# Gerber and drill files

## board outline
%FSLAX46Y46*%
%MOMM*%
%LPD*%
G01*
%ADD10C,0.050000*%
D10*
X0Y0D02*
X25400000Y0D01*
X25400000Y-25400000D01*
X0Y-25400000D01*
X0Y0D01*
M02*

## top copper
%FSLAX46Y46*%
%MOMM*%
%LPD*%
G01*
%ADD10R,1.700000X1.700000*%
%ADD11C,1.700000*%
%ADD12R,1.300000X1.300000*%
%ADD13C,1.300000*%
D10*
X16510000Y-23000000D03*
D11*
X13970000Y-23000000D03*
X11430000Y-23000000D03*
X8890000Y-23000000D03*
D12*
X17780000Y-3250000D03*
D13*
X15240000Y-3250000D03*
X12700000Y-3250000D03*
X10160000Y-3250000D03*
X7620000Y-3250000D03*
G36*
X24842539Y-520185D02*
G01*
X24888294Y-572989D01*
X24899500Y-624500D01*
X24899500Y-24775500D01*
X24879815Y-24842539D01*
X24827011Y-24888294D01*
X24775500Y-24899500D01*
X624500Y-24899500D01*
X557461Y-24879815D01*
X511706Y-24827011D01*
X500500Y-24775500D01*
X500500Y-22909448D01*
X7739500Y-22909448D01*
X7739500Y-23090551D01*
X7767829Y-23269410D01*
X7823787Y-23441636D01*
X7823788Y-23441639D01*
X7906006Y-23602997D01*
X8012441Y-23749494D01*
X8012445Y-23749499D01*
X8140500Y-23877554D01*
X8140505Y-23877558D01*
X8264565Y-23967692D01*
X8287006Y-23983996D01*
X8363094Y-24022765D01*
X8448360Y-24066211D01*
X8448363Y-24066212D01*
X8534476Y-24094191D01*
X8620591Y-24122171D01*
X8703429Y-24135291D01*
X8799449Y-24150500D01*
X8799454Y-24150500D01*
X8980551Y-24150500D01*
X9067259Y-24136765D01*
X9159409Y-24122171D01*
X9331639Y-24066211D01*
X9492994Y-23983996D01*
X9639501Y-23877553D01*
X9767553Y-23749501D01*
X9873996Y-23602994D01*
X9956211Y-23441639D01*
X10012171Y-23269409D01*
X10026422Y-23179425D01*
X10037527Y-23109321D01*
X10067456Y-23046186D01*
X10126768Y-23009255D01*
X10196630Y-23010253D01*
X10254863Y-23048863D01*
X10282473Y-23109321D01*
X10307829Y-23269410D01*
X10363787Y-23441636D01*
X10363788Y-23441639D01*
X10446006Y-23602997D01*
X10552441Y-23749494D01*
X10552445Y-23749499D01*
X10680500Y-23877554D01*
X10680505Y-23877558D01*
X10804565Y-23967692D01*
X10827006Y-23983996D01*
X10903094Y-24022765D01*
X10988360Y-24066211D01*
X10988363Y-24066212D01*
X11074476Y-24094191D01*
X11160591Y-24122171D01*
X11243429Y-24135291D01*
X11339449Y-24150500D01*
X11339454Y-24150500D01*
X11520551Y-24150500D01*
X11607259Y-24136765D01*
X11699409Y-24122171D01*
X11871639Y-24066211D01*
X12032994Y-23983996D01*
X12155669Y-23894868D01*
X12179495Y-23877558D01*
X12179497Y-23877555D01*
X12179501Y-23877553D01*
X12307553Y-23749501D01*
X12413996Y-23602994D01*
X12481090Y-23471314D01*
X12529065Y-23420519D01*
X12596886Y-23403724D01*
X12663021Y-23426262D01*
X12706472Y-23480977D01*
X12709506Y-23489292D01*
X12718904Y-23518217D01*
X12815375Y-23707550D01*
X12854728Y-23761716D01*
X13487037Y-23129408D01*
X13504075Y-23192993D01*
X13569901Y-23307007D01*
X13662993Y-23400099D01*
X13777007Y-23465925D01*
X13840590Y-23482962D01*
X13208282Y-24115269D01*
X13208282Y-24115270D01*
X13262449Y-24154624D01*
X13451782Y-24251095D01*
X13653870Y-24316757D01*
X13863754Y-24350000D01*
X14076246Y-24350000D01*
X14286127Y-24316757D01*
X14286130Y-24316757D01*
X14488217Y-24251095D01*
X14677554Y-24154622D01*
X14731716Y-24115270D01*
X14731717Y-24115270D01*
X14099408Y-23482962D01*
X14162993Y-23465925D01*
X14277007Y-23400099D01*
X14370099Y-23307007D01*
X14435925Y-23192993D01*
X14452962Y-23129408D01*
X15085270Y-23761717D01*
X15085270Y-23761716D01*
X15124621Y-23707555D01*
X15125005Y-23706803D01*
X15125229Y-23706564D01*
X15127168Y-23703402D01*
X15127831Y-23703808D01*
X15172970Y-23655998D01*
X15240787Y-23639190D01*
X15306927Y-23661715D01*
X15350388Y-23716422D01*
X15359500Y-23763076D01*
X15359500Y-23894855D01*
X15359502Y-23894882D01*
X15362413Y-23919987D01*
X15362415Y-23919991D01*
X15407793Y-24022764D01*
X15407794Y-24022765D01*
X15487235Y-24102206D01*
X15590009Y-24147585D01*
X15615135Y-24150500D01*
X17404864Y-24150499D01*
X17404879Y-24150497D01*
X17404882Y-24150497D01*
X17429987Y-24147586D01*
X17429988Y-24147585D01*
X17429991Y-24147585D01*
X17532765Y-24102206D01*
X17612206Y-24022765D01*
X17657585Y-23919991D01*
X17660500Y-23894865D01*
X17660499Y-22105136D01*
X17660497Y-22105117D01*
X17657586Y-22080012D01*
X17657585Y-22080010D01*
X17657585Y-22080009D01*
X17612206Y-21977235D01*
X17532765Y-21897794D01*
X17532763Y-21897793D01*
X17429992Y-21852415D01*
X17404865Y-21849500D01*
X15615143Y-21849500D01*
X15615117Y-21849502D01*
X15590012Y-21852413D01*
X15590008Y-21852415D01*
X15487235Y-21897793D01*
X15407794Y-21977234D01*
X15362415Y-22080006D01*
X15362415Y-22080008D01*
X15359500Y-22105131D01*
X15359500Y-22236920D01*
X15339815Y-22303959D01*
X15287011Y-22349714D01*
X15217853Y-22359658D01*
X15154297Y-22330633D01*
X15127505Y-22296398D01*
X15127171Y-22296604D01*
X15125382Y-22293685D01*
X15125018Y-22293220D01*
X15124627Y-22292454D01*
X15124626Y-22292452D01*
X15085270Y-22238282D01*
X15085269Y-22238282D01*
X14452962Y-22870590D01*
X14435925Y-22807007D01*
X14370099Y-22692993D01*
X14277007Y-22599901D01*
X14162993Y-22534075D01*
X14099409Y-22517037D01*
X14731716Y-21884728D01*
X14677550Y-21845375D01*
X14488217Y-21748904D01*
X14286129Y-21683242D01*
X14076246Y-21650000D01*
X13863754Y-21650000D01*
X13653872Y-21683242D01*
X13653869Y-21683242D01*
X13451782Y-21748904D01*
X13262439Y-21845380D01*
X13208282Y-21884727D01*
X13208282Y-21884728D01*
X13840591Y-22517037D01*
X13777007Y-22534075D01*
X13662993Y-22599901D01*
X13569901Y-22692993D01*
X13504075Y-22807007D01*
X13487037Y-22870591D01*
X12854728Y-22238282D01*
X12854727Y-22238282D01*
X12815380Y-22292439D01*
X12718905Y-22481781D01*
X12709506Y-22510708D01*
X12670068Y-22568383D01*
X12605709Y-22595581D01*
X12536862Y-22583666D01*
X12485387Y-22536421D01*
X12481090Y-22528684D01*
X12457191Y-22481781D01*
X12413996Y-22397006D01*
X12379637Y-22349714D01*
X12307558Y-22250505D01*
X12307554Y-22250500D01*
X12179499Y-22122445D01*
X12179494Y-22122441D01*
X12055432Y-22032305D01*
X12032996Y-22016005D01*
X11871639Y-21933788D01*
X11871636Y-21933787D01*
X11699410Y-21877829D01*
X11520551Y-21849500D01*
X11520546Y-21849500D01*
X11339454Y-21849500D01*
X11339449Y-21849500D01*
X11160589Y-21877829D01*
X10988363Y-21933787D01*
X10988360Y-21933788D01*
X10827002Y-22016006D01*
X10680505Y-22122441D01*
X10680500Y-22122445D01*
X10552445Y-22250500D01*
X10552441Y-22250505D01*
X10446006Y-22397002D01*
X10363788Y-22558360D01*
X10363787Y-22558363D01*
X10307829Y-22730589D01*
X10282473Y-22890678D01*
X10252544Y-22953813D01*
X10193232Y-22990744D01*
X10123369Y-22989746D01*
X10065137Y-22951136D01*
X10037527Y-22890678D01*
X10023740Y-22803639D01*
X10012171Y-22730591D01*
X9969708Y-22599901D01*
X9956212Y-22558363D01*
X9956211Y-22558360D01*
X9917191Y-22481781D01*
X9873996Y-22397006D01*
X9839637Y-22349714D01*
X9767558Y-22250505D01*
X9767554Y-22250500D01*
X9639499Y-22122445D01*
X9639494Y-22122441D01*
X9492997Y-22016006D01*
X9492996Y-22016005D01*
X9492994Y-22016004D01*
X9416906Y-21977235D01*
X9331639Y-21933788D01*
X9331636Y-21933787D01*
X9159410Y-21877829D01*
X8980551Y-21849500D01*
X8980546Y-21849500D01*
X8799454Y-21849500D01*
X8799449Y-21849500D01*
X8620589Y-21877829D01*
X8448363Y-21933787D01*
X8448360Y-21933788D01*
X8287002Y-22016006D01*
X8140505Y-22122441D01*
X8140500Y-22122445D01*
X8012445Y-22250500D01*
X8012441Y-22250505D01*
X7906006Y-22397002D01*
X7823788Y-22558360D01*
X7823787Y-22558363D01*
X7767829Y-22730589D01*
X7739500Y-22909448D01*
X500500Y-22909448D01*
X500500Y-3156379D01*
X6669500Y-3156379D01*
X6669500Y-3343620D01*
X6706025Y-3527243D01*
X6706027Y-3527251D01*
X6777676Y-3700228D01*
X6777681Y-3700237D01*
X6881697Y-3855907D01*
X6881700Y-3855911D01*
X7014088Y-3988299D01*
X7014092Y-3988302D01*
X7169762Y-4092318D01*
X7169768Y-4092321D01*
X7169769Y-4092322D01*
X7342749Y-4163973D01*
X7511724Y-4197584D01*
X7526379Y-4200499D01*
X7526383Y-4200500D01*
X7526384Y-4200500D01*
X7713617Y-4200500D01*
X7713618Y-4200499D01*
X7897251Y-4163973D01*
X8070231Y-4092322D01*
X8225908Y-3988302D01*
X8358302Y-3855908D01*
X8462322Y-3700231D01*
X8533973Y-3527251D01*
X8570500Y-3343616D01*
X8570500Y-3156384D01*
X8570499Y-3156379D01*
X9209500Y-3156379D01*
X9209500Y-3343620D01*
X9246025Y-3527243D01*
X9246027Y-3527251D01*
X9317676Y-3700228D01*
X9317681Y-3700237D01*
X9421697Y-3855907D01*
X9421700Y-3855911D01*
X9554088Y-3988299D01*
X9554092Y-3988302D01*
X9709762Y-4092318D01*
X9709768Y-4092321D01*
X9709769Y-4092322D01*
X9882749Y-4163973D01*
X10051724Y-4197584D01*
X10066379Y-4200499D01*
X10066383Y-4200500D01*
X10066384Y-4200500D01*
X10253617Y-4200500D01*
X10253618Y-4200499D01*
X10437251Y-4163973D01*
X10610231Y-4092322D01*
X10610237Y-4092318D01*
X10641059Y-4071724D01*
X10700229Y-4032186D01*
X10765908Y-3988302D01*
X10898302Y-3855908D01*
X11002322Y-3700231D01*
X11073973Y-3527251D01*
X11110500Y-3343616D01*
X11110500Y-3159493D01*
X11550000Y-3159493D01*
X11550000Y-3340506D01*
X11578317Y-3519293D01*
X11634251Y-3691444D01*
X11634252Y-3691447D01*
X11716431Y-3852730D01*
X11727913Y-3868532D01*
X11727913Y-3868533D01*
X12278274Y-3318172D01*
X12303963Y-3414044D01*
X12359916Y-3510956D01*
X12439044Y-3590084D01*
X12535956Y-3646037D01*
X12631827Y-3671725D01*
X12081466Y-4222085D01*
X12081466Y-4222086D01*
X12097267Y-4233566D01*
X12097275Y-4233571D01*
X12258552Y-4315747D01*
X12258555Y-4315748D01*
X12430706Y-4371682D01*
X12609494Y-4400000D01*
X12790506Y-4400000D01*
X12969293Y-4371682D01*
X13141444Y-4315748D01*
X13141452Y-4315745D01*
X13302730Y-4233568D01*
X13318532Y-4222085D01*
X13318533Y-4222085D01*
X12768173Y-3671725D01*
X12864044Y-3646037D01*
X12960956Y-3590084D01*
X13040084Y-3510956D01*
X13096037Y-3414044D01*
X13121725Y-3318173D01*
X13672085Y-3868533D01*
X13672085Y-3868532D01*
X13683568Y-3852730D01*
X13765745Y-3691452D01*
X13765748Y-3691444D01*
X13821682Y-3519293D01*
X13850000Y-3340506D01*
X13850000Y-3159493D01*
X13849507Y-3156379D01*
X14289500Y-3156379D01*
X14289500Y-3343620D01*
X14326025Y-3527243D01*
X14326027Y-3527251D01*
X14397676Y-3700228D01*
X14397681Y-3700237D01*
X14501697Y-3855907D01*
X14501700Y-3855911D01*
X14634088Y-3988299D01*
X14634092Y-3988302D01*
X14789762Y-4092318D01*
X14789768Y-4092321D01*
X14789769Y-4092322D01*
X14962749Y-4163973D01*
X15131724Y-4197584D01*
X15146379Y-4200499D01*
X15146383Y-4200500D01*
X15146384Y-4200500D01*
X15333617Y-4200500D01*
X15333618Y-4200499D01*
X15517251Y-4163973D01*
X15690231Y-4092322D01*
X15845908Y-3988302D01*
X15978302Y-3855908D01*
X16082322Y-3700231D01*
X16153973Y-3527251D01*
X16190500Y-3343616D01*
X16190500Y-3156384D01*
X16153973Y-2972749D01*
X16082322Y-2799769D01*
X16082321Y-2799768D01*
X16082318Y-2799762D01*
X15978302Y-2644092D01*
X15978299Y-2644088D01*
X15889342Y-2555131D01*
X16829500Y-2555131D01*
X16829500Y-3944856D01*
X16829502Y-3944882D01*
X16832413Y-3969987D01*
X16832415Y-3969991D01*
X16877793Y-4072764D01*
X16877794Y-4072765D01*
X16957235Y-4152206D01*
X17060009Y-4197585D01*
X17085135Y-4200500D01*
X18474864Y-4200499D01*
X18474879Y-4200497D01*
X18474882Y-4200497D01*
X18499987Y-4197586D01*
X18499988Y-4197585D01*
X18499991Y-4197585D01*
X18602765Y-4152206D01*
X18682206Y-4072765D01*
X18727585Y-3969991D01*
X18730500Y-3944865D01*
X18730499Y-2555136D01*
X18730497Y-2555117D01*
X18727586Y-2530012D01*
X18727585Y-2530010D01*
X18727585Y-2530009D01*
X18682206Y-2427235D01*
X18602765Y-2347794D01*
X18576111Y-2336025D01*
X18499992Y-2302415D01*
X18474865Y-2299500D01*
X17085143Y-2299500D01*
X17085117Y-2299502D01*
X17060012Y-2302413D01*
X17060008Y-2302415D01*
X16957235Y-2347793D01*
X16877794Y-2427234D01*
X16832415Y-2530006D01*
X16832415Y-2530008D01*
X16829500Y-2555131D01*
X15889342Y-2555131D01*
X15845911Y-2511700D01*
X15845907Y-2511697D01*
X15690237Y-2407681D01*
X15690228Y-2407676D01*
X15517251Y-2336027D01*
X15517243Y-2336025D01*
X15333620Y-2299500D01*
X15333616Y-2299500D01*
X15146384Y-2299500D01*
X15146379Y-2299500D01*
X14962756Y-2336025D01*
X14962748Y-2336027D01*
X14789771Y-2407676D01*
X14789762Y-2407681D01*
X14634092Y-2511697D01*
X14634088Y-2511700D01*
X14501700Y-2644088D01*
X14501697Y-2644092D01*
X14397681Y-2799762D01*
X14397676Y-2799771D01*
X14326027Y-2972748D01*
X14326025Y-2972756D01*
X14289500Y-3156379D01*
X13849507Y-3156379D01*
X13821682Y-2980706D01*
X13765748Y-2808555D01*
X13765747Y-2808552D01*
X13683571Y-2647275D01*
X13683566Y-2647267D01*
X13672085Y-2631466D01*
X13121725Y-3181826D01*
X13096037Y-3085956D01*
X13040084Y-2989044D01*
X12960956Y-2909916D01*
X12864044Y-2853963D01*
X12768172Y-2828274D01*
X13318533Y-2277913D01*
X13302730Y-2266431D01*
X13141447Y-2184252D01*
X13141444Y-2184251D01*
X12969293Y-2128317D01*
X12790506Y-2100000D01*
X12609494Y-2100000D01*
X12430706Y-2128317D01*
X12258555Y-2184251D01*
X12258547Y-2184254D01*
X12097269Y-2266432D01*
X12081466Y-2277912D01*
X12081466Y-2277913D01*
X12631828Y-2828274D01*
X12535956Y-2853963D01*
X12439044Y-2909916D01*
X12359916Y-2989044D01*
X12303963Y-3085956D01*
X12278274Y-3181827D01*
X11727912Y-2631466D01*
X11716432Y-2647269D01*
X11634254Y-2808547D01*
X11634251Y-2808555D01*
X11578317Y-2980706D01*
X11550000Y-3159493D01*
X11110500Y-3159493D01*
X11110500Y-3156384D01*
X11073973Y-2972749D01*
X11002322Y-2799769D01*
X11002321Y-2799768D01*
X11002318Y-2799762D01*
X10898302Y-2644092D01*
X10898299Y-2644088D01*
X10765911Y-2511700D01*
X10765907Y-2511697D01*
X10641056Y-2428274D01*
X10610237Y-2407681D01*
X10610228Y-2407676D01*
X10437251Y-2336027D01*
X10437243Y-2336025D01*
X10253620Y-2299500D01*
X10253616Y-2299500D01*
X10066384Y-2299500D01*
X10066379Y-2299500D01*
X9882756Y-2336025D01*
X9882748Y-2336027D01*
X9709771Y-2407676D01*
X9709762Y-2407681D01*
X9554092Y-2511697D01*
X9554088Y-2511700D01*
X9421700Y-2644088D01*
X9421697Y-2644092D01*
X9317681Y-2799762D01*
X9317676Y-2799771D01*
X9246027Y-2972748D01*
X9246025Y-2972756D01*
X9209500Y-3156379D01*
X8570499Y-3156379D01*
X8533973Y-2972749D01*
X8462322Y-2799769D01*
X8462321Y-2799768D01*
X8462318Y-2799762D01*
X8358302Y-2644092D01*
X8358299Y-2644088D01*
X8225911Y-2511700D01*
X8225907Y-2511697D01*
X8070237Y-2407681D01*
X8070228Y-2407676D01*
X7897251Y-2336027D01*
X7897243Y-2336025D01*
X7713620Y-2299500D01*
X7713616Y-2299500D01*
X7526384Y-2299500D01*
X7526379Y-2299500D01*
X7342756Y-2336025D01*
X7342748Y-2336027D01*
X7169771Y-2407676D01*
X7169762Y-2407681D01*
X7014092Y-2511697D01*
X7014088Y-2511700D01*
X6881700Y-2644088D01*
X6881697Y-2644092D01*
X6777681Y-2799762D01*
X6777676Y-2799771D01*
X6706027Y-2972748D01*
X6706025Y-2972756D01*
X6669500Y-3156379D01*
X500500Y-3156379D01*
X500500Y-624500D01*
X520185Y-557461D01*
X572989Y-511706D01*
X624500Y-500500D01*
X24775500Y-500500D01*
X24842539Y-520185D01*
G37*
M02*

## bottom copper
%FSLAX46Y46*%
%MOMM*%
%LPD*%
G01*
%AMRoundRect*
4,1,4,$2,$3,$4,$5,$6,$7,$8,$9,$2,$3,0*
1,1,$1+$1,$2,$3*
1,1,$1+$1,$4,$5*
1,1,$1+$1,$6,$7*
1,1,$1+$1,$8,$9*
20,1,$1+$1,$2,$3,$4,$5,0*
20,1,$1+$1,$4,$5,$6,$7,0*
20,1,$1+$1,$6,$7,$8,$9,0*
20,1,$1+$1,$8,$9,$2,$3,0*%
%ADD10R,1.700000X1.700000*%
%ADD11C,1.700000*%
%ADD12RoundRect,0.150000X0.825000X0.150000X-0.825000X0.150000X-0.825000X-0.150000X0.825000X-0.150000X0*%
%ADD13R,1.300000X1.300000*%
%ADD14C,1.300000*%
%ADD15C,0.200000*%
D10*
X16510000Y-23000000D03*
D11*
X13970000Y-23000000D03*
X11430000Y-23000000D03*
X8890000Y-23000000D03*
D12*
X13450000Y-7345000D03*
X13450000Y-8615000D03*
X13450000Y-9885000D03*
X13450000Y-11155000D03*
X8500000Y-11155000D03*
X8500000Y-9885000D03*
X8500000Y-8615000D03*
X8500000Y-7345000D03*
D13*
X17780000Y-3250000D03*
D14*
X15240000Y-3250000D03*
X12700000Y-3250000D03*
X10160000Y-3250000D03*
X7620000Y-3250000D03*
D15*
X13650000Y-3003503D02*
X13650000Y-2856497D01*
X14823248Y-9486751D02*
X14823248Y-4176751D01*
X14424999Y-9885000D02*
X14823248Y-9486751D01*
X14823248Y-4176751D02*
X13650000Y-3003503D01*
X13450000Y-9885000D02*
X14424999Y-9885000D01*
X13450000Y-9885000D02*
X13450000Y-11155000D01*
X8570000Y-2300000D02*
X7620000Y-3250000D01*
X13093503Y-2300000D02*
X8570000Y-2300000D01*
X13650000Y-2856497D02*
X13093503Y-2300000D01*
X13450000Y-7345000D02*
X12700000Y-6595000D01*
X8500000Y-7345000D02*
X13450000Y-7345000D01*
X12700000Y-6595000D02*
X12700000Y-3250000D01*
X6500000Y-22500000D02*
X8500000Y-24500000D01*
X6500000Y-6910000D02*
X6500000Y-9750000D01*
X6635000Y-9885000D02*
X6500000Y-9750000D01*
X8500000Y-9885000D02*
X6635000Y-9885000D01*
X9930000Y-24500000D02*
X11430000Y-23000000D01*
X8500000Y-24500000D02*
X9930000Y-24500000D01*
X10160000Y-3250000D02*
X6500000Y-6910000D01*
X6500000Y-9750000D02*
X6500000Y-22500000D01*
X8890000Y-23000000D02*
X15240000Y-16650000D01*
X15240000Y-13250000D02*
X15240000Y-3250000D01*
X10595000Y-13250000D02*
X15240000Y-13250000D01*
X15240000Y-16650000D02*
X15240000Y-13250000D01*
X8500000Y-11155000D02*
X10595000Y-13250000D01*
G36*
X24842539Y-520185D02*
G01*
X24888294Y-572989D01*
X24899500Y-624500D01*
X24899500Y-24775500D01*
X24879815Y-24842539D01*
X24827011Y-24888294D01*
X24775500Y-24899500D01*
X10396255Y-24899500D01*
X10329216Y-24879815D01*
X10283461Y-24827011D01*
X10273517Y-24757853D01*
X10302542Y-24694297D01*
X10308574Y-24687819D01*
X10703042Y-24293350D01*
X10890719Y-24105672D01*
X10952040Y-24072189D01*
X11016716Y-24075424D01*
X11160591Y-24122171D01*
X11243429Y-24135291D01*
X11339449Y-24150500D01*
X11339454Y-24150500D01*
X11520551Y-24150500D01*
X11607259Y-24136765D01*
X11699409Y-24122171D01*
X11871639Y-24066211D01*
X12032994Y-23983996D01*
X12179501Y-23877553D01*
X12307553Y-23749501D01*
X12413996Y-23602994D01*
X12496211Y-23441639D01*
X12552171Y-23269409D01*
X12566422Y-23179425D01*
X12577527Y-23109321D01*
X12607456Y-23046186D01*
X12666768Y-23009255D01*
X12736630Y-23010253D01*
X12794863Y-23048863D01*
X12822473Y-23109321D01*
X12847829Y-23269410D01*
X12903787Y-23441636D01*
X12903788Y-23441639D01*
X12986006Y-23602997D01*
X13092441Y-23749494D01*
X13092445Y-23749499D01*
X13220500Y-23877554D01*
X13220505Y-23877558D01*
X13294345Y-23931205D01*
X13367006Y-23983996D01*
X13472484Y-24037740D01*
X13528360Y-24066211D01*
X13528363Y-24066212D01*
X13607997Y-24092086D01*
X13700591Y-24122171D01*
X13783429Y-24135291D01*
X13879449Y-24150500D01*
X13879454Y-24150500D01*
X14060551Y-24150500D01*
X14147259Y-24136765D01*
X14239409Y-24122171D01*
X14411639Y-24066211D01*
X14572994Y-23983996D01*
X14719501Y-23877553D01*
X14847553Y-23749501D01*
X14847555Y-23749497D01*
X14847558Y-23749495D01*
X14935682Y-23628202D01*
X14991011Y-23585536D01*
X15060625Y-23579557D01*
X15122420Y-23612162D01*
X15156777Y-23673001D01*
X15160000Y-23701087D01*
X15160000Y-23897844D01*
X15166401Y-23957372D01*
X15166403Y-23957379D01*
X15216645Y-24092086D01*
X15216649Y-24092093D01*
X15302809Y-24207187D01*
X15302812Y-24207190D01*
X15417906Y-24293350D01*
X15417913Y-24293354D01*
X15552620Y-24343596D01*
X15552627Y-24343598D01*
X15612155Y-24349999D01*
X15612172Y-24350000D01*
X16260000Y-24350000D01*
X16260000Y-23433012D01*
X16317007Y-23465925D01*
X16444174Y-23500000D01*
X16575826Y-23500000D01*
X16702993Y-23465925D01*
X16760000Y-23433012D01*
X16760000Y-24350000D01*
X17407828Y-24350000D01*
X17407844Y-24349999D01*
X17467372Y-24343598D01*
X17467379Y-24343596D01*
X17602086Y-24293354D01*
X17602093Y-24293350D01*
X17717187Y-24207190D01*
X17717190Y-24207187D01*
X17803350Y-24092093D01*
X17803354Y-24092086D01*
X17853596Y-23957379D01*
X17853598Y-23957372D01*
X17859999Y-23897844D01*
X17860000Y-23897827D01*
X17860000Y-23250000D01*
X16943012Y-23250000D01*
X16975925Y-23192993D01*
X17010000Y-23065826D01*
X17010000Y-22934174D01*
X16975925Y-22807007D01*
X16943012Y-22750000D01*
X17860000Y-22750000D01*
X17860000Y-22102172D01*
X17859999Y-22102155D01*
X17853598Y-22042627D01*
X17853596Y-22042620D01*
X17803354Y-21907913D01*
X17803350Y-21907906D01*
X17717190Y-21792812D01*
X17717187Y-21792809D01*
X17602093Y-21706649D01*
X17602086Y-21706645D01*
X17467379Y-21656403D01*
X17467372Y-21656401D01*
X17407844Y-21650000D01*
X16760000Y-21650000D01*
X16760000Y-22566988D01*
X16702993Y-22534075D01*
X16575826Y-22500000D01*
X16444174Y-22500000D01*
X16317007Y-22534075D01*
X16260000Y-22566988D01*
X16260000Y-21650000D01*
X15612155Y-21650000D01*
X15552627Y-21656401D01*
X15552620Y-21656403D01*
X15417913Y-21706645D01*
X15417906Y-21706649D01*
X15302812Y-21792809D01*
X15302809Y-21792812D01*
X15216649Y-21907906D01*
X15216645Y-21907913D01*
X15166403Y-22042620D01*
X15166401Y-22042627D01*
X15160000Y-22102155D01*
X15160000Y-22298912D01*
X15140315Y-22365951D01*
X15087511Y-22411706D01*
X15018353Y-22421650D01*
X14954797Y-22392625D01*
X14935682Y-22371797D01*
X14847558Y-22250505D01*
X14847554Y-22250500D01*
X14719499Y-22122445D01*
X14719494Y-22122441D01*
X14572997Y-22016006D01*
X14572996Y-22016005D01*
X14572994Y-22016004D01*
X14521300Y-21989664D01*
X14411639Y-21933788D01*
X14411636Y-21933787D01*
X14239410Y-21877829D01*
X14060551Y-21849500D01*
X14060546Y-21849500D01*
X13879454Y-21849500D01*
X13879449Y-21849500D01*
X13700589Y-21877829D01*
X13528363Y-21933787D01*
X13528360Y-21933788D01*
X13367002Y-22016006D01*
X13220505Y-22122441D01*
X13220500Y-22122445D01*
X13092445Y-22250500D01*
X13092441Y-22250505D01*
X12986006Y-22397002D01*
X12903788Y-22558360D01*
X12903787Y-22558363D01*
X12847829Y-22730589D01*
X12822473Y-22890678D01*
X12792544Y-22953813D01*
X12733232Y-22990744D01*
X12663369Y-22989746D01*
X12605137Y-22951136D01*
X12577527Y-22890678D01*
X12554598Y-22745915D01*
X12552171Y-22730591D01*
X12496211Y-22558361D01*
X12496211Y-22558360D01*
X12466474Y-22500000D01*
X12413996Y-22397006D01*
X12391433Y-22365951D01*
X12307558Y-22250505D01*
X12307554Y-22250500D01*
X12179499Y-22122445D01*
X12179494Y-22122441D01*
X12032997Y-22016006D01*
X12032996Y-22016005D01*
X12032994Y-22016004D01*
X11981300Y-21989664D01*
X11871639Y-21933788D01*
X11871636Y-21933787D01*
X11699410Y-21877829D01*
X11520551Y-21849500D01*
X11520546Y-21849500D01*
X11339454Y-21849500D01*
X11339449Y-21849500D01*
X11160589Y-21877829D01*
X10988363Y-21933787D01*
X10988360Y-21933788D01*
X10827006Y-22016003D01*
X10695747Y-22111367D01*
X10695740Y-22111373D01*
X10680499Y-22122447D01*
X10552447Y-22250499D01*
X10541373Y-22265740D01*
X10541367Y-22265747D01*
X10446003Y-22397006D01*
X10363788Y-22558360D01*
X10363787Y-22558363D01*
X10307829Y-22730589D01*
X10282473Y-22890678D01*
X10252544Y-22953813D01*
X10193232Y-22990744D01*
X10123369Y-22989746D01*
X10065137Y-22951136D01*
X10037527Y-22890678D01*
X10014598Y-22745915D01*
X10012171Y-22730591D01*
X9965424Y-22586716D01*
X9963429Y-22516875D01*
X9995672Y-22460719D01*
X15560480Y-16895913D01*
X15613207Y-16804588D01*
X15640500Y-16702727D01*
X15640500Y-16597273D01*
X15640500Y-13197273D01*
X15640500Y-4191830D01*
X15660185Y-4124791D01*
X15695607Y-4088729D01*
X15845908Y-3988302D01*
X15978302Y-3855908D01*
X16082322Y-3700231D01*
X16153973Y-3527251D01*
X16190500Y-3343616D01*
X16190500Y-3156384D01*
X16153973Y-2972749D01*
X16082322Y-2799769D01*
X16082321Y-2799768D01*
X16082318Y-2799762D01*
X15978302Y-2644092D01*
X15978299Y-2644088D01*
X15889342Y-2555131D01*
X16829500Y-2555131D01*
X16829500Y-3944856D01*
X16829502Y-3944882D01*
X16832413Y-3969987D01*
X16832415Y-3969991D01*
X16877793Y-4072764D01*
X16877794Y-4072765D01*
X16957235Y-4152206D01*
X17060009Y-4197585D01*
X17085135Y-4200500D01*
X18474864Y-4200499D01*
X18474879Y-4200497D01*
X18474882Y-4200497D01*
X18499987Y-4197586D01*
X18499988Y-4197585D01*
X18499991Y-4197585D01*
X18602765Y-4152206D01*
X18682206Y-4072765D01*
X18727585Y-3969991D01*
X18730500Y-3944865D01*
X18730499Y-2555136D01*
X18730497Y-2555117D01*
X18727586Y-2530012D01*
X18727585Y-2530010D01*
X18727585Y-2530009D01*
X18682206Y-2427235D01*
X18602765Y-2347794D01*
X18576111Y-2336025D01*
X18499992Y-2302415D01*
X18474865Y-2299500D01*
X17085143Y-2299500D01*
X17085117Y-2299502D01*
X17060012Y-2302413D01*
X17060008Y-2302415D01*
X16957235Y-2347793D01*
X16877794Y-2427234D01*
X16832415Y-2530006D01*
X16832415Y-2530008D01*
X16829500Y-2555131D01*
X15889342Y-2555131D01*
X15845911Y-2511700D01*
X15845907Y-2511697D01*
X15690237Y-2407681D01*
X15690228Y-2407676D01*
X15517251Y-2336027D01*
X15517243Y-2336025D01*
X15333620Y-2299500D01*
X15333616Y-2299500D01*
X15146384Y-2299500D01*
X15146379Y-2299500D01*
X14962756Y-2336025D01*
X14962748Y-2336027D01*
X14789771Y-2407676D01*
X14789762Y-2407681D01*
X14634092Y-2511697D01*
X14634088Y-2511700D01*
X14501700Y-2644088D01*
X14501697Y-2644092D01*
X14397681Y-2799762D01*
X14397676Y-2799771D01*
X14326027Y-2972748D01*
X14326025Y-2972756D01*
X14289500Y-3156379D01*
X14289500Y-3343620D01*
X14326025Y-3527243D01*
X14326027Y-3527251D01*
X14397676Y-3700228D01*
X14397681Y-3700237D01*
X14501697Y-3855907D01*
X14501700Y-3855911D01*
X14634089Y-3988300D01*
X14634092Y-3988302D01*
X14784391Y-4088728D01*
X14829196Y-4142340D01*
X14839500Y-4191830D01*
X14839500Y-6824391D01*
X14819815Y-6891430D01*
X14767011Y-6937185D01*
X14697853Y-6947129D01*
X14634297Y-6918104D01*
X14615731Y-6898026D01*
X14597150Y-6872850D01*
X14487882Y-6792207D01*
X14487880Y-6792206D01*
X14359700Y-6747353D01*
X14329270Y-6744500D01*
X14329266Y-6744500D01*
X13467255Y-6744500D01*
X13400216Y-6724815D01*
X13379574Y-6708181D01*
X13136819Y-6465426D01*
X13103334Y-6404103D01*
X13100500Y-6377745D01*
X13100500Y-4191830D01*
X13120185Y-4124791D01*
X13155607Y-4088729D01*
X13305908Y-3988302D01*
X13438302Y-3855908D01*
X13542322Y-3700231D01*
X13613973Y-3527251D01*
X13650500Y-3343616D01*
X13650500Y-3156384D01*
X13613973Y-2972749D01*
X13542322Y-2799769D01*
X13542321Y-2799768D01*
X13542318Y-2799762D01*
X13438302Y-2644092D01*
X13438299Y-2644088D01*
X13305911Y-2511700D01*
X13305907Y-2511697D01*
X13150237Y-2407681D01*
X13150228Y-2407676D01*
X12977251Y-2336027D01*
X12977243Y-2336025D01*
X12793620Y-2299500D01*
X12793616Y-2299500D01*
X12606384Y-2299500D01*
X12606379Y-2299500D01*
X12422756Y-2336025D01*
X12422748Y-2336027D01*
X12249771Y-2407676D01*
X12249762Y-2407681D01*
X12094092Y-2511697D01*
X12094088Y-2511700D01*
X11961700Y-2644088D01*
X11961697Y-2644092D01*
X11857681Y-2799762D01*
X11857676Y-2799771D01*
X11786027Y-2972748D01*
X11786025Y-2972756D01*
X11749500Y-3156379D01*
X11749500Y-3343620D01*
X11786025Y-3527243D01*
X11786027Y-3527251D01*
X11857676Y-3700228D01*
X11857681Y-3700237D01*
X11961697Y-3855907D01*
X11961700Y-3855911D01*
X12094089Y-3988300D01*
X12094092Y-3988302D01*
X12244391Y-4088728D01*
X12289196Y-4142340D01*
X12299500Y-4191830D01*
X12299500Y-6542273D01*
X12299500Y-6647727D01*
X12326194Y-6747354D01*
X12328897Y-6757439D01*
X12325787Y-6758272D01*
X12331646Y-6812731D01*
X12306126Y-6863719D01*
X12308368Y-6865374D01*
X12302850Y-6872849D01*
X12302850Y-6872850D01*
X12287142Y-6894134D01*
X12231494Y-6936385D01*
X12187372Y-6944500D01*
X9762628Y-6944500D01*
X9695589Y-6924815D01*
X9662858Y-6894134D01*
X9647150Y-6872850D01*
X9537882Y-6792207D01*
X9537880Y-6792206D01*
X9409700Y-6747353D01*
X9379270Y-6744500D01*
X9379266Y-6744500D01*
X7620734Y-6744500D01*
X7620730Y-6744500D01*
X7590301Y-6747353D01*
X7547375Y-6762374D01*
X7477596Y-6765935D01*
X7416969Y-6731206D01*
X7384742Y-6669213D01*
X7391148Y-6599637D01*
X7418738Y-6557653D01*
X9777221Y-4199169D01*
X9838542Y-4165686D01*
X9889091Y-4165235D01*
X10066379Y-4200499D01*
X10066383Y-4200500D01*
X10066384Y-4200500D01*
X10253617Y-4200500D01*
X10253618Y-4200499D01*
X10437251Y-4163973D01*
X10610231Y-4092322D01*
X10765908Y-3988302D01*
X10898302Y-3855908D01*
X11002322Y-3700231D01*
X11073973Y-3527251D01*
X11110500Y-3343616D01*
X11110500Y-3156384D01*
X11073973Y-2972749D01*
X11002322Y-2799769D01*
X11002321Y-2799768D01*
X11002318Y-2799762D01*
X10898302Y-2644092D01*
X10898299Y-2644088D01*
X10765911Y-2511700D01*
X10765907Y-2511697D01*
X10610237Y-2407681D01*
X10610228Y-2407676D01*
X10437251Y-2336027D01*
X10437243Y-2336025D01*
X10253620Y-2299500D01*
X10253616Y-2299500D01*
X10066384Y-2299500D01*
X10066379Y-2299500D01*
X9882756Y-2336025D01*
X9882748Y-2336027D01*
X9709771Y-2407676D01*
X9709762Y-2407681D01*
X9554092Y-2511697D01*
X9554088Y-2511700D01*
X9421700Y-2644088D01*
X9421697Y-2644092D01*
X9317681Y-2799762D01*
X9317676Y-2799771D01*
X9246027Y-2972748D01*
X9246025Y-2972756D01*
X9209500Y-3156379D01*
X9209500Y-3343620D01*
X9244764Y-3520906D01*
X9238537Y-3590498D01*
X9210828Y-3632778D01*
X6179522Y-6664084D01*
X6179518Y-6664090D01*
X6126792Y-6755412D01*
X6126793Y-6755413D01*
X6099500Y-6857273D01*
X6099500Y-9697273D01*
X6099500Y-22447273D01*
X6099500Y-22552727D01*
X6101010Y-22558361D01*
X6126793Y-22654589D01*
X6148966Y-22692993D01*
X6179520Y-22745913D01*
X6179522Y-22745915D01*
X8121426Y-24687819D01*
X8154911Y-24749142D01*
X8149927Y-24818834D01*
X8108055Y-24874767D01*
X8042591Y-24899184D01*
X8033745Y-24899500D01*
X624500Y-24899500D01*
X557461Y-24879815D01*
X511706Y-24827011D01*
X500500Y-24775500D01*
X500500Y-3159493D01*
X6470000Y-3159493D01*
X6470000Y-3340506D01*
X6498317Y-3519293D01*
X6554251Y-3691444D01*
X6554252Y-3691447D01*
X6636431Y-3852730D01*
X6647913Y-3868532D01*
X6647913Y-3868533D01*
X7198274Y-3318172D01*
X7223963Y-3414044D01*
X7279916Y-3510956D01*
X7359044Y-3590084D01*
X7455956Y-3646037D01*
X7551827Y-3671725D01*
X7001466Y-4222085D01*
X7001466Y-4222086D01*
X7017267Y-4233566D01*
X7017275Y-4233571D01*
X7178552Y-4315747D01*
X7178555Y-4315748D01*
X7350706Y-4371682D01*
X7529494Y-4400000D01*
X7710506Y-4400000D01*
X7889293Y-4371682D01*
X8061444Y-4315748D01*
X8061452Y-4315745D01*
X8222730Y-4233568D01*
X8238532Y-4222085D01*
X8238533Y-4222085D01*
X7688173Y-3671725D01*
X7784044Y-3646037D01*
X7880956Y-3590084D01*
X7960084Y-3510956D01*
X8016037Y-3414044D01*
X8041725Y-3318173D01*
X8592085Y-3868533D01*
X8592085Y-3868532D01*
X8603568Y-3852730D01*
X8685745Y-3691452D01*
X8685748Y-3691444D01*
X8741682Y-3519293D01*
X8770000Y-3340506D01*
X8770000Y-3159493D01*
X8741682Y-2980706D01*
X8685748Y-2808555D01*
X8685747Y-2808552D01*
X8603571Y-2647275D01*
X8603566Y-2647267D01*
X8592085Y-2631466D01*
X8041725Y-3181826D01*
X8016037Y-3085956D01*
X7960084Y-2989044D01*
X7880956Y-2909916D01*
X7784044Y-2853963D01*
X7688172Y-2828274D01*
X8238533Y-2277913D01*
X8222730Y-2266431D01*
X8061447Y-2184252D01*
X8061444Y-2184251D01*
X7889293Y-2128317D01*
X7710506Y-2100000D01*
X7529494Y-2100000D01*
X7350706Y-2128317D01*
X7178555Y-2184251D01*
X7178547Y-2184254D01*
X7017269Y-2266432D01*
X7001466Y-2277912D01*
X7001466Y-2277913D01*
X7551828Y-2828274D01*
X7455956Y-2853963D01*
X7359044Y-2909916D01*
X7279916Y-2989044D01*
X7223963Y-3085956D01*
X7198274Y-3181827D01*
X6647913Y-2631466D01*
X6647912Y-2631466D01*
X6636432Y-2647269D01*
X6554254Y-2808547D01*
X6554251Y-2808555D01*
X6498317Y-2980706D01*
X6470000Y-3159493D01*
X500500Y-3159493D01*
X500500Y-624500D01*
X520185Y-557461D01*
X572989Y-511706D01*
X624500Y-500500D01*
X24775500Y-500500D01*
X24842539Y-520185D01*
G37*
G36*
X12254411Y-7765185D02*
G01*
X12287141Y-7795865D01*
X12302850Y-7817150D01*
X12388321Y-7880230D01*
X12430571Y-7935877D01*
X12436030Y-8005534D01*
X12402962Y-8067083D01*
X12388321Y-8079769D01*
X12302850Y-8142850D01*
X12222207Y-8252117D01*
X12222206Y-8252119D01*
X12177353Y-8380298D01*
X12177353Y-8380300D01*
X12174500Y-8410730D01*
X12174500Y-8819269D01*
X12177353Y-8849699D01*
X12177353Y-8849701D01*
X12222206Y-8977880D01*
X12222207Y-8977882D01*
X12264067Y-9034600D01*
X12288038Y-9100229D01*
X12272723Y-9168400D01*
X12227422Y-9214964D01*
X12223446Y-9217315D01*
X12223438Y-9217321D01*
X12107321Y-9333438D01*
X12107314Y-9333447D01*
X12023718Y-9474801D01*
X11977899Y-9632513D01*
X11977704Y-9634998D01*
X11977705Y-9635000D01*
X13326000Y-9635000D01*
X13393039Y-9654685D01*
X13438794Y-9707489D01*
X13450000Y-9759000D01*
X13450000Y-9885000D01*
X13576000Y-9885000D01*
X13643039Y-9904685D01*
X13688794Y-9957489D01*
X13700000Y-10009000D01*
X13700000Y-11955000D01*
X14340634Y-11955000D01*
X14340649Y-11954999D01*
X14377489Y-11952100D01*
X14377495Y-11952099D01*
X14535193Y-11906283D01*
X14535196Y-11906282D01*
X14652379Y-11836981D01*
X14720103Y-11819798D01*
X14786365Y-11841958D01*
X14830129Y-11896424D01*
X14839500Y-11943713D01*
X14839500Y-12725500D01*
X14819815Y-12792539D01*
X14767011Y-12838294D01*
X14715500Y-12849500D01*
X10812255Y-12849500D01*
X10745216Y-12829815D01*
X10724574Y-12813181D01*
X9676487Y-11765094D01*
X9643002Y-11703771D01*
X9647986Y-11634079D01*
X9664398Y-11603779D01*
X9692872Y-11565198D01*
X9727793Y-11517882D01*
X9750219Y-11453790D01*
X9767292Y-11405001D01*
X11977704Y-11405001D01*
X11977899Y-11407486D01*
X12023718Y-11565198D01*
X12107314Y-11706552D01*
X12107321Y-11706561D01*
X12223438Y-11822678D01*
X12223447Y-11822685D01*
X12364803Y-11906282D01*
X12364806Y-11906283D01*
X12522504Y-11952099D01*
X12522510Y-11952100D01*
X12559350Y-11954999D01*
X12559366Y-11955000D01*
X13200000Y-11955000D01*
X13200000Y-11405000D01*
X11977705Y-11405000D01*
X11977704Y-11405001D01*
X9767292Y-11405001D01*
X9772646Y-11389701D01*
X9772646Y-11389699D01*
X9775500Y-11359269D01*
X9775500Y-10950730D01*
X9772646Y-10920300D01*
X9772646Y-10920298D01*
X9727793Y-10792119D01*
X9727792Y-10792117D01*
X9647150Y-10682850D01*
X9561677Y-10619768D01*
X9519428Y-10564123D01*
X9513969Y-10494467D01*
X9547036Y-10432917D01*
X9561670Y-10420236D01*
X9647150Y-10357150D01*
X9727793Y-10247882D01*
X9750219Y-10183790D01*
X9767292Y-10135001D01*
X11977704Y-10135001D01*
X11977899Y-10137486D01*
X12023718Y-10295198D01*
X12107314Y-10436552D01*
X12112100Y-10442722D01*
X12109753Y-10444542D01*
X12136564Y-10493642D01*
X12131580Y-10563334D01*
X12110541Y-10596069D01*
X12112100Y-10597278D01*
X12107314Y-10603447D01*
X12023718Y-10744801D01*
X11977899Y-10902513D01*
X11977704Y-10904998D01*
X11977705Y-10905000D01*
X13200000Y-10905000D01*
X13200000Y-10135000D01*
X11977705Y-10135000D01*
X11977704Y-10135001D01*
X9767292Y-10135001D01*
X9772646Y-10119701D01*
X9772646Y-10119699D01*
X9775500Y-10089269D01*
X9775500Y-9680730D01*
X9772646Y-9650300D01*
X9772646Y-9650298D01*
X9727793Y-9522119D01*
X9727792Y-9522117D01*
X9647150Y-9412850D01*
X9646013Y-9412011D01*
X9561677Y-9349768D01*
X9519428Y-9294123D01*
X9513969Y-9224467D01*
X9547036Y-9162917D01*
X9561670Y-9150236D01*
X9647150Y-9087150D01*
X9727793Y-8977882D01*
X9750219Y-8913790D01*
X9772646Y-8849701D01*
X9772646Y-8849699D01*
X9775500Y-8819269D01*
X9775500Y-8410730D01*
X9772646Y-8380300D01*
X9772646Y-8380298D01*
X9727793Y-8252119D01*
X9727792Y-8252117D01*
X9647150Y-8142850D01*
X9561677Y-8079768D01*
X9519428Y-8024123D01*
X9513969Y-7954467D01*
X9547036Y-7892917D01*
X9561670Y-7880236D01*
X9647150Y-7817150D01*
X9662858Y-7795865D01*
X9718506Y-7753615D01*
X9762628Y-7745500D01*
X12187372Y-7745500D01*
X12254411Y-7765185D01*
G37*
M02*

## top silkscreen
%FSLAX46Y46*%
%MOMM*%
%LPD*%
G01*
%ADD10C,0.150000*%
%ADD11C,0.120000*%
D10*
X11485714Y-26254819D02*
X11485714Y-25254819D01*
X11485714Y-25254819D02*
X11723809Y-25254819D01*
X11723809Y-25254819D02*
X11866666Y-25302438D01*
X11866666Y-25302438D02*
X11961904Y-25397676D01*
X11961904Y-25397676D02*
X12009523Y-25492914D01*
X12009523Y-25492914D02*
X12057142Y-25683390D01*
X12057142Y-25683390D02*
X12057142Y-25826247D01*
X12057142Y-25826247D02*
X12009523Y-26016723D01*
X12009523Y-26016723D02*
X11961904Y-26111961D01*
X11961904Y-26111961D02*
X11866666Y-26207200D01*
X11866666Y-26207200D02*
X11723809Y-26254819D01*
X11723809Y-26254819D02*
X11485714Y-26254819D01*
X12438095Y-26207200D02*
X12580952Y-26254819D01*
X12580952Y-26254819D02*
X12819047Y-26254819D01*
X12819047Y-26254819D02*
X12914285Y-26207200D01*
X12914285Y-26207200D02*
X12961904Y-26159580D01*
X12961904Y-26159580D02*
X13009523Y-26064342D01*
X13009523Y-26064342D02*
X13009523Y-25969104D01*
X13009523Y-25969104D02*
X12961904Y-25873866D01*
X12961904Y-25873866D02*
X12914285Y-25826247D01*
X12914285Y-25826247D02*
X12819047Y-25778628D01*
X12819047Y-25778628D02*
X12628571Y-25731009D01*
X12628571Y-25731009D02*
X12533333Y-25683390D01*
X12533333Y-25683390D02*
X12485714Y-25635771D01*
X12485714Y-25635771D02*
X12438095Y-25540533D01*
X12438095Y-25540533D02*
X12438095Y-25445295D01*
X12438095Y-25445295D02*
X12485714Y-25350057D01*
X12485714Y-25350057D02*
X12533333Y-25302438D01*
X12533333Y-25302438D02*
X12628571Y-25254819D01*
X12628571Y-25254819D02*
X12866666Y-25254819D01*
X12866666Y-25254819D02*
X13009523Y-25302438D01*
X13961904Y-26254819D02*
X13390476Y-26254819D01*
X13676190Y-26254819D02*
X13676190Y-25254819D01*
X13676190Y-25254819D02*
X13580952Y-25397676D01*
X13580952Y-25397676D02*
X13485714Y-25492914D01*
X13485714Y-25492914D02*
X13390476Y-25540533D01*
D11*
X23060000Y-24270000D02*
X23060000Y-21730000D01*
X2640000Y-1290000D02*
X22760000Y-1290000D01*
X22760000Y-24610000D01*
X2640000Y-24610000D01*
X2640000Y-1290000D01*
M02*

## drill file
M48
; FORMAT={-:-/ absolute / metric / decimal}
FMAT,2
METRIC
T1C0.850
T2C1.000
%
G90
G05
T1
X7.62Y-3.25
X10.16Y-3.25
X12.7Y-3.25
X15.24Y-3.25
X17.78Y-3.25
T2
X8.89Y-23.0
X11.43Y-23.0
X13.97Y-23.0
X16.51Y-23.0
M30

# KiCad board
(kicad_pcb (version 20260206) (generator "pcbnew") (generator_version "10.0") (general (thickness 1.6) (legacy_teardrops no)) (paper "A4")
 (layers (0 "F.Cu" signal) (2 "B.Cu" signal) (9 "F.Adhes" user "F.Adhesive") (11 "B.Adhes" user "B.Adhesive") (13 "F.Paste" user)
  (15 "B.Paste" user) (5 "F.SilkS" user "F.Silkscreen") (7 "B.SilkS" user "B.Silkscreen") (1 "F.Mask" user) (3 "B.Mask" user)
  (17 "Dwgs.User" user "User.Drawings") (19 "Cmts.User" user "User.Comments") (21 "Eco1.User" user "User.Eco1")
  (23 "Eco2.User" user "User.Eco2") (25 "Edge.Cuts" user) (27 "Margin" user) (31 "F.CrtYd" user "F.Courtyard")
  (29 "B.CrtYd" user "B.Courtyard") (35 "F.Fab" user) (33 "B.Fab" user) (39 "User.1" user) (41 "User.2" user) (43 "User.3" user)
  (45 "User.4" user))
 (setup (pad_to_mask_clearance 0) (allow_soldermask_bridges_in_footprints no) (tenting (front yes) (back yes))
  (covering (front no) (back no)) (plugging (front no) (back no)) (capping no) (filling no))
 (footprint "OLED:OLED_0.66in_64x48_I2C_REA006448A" (layer "F.Cu") (at 16.51 23 180)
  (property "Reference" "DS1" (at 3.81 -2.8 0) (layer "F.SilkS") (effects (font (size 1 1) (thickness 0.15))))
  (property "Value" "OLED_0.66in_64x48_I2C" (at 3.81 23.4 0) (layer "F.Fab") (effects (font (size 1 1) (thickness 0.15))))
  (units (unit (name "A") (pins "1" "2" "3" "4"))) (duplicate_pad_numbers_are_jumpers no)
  (fp_line (start -6.55 -1.27) (end -6.55 1.27) (stroke (width 0.12) (type solid)) (layer "F.SilkS"))
  (fp_rect (start -6.25 -1.61) (end 13.87 21.71) (stroke (width 0.12) (type solid)) (fill no) (layer "F.SilkS"))
  (pad "1" thru_hole rect (at 0 0 180) (size 1.7 1.7) (drill 1) (layers "*.Cu" "*.Mask") (remove_unused_layers no) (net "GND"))
  (pad "2" thru_hole circle (at 2.54 0 180) (size 1.7 1.7) (drill 1) (layers "*.Cu" "*.Mask") (remove_unused_layers no) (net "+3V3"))
  (pad "3" thru_hole circle (at 5.08 0 180) (size 1.7 1.7) (drill 1) (layers "*.Cu" "*.Mask") (remove_unused_layers no) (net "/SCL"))
  (pad "4" thru_hole circle (at 7.62 0 180) (size 1.7 1.7) (drill 1) (layers "*.Cu" "*.Mask") (remove_unused_layers no) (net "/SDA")))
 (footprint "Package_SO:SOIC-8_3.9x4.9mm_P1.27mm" (layer "B.Cu") (at 10.975 9.25 180)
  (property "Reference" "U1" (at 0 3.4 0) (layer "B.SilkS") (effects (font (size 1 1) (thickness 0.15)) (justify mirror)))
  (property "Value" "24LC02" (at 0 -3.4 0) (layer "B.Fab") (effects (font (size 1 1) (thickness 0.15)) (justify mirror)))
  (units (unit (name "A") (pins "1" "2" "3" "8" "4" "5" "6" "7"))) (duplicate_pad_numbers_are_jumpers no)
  (pad "1" smd roundrect (at -2.475 1.905 180) (size 1.95 0.6) (layers "B.Cu" "B.Mask" "B.Paste") (roundrect_rratio 0.25) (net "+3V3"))
  (pad "2" smd roundrect (at -2.475 0.635 180) (size 1.95 0.6) (layers "B.Cu" "B.Mask" "B.Paste") (roundrect_rratio 0.25)
   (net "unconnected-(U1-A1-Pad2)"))
  (pad "3" smd roundrect (at -2.475 -0.635 180) (size 1.95 0.6) (layers "B.Cu" "B.Mask" "B.Paste") (roundrect_rratio 0.25) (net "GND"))
  (pad "4" smd roundrect (at -2.475 -1.905 180) (size 1.95 0.6) (layers "B.Cu" "B.Mask" "B.Paste") (roundrect_rratio 0.25) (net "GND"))
  (pad "5" smd roundrect (at 2.475 -1.905 180) (size 1.95 0.6) (layers "B.Cu" "B.Mask" "B.Paste") (roundrect_rratio 0.25) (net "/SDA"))
  (pad "6" smd roundrect (at 2.475 -0.635 180) (size 1.95 0.6) (layers "B.Cu" "B.Mask" "B.Paste") (roundrect_rratio 0.25) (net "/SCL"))
  (pad "7" smd roundrect (at 2.475 0.635 180) (size 1.95 0.6) (layers "B.Cu" "B.Mask" "B.Paste") (roundrect_rratio 0.25)
   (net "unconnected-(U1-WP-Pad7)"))
  (pad "8" smd roundrect (at 2.475 1.905 180) (size 1.95 0.6) (layers "B.Cu" "B.Mask" "B.Paste") (roundrect_rratio 0.25) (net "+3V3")))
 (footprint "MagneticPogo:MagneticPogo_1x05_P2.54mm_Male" (layer "B.Cu") (at 12.7 3.25 180)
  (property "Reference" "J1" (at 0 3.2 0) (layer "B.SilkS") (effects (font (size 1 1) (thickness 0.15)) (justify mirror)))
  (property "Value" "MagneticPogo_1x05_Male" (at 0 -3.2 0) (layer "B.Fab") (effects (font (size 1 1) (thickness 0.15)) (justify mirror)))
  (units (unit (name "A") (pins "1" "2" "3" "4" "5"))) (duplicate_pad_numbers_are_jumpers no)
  (pad "1" thru_hole rect (at -5.08 0 180) (size 1.3 1.3) (drill 0.85) (layers "*.Cu" "*.Mask") (remove_unused_layers no) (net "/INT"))
  (pad "2" thru_hole circle (at -2.54 0 180) (size 1.3 1.3) (drill 0.85) (layers "*.Cu" "*.Mask") (remove_unused_layers no) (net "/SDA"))
  (pad "3" thru_hole circle (at 0 0 180) (size 1.3 1.3) (drill 0.85) (layers "*.Cu" "*.Mask") (remove_unused_layers no) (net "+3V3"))
  (pad "4" thru_hole circle (at 2.54 0 180) (size 1.3 1.3) (drill 0.85) (layers "*.Cu" "*.Mask") (remove_unused_layers no) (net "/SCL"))
  (pad "5" thru_hole circle (at 5.08 0 180) (size 1.3 1.3) (drill 0.85) (layers "*.Cu" "*.Mask") (remove_unused_layers no) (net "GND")))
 (gr_rect (start 0 0) (end 25.4 25.4) (stroke (width 0.05) (type default)) (fill no) (layer "Edge.Cuts"))
 (segment (start 13.65 3.003503) (end 13.65 2.856497) (width 0.2) (layer "B.Cu") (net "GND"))
 (segment (start 14.823248 9.486751) (end 14.823248 4.176751) (width 0.2) (layer "B.Cu") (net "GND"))
 (segment (start 14.424999 9.885) (end 14.823248 9.486751) (width 0.2) (layer "B.Cu") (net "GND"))
 (segment (start 14.823248 4.176751) (end 13.65 3.003503) (width 0.2) (layer "B.Cu") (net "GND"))
 (segment (start 13.45 9.885) (end 14.424999 9.885) (width 0.2) (layer "B.Cu") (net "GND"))
 (segment (start 13.45 9.885) (end 13.45 11.155) (width 0.2) (layer "B.Cu") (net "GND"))
 (segment (start 8.57 2.3) (end 7.62 3.25) (width 0.2) (layer "B.Cu") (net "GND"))
 (segment (start 13.093503 2.3) (end 8.57 2.3) (width 0.2) (layer "B.Cu") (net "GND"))
 (segment (start 13.65 2.856497) (end 13.093503 2.3) (width 0.2) (layer "B.Cu") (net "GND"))
 (segment (start 13.45 7.345) (end 12.7 6.595) (width 0.2) (layer "B.Cu") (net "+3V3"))
 (segment (start 8.5 7.345) (end 13.45 7.345) (width 0.2) (layer "B.Cu") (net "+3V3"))
 (segment (start 12.7 6.595) (end 12.7 3.25) (width 0.2) (layer "B.Cu") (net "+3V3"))
 (segment (start 6.5 22.5) (end 8.5 24.5) (width 0.2) (layer "B.Cu") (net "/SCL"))
 (segment (start 6.5 6.91) (end 6.5 9.75) (width 0.2) (layer "B.Cu") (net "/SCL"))
 (segment (start 6.635 9.885) (end 6.5 9.75) (width 0.2) (layer "B.Cu") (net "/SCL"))
 (segment (start 8.5 9.885) (end 6.635 9.885) (width 0.2) (layer "B.Cu") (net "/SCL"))
 (segment (start 9.93 24.5) (end 11.43 23) (width 0.2) (layer "B.Cu") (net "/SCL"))
 (segment (start 8.5 24.5) (end 9.93 24.5) (width 0.2) (layer "B.Cu") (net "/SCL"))
 (segment (start 10.16 3.25) (end 6.5 6.91) (width 0.2) (layer "B.Cu") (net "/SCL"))
 (segment (start 6.5 9.75) (end 6.5 22.5) (width 0.2) (layer "B.Cu") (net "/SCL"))
 (segment (start 8.89 23) (end 15.24 16.65) (width 0.2) (layer "B.Cu") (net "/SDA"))
 (segment (start 15.24 13.25) (end 15.24 3.25) (width 0.2) (layer "B.Cu") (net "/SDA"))
 (segment (start 10.595 13.25) (end 15.24 13.25) (width 0.2) (layer "B.Cu") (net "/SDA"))
 (segment (start 15.24 16.65) (end 15.24 13.25) (width 0.2) (layer "B.Cu") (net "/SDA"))
 (segment (start 8.5 11.155) (end 10.595 13.25) (width 0.2) (layer "B.Cu") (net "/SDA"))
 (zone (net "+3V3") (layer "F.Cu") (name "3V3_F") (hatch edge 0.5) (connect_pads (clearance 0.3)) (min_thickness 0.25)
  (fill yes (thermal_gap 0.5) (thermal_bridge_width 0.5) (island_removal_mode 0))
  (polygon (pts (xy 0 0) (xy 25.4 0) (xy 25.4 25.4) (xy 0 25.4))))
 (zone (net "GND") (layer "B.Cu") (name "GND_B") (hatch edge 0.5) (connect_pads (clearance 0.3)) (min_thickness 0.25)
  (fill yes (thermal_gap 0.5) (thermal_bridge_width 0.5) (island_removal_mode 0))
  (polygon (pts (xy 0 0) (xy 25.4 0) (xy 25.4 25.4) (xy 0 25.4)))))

